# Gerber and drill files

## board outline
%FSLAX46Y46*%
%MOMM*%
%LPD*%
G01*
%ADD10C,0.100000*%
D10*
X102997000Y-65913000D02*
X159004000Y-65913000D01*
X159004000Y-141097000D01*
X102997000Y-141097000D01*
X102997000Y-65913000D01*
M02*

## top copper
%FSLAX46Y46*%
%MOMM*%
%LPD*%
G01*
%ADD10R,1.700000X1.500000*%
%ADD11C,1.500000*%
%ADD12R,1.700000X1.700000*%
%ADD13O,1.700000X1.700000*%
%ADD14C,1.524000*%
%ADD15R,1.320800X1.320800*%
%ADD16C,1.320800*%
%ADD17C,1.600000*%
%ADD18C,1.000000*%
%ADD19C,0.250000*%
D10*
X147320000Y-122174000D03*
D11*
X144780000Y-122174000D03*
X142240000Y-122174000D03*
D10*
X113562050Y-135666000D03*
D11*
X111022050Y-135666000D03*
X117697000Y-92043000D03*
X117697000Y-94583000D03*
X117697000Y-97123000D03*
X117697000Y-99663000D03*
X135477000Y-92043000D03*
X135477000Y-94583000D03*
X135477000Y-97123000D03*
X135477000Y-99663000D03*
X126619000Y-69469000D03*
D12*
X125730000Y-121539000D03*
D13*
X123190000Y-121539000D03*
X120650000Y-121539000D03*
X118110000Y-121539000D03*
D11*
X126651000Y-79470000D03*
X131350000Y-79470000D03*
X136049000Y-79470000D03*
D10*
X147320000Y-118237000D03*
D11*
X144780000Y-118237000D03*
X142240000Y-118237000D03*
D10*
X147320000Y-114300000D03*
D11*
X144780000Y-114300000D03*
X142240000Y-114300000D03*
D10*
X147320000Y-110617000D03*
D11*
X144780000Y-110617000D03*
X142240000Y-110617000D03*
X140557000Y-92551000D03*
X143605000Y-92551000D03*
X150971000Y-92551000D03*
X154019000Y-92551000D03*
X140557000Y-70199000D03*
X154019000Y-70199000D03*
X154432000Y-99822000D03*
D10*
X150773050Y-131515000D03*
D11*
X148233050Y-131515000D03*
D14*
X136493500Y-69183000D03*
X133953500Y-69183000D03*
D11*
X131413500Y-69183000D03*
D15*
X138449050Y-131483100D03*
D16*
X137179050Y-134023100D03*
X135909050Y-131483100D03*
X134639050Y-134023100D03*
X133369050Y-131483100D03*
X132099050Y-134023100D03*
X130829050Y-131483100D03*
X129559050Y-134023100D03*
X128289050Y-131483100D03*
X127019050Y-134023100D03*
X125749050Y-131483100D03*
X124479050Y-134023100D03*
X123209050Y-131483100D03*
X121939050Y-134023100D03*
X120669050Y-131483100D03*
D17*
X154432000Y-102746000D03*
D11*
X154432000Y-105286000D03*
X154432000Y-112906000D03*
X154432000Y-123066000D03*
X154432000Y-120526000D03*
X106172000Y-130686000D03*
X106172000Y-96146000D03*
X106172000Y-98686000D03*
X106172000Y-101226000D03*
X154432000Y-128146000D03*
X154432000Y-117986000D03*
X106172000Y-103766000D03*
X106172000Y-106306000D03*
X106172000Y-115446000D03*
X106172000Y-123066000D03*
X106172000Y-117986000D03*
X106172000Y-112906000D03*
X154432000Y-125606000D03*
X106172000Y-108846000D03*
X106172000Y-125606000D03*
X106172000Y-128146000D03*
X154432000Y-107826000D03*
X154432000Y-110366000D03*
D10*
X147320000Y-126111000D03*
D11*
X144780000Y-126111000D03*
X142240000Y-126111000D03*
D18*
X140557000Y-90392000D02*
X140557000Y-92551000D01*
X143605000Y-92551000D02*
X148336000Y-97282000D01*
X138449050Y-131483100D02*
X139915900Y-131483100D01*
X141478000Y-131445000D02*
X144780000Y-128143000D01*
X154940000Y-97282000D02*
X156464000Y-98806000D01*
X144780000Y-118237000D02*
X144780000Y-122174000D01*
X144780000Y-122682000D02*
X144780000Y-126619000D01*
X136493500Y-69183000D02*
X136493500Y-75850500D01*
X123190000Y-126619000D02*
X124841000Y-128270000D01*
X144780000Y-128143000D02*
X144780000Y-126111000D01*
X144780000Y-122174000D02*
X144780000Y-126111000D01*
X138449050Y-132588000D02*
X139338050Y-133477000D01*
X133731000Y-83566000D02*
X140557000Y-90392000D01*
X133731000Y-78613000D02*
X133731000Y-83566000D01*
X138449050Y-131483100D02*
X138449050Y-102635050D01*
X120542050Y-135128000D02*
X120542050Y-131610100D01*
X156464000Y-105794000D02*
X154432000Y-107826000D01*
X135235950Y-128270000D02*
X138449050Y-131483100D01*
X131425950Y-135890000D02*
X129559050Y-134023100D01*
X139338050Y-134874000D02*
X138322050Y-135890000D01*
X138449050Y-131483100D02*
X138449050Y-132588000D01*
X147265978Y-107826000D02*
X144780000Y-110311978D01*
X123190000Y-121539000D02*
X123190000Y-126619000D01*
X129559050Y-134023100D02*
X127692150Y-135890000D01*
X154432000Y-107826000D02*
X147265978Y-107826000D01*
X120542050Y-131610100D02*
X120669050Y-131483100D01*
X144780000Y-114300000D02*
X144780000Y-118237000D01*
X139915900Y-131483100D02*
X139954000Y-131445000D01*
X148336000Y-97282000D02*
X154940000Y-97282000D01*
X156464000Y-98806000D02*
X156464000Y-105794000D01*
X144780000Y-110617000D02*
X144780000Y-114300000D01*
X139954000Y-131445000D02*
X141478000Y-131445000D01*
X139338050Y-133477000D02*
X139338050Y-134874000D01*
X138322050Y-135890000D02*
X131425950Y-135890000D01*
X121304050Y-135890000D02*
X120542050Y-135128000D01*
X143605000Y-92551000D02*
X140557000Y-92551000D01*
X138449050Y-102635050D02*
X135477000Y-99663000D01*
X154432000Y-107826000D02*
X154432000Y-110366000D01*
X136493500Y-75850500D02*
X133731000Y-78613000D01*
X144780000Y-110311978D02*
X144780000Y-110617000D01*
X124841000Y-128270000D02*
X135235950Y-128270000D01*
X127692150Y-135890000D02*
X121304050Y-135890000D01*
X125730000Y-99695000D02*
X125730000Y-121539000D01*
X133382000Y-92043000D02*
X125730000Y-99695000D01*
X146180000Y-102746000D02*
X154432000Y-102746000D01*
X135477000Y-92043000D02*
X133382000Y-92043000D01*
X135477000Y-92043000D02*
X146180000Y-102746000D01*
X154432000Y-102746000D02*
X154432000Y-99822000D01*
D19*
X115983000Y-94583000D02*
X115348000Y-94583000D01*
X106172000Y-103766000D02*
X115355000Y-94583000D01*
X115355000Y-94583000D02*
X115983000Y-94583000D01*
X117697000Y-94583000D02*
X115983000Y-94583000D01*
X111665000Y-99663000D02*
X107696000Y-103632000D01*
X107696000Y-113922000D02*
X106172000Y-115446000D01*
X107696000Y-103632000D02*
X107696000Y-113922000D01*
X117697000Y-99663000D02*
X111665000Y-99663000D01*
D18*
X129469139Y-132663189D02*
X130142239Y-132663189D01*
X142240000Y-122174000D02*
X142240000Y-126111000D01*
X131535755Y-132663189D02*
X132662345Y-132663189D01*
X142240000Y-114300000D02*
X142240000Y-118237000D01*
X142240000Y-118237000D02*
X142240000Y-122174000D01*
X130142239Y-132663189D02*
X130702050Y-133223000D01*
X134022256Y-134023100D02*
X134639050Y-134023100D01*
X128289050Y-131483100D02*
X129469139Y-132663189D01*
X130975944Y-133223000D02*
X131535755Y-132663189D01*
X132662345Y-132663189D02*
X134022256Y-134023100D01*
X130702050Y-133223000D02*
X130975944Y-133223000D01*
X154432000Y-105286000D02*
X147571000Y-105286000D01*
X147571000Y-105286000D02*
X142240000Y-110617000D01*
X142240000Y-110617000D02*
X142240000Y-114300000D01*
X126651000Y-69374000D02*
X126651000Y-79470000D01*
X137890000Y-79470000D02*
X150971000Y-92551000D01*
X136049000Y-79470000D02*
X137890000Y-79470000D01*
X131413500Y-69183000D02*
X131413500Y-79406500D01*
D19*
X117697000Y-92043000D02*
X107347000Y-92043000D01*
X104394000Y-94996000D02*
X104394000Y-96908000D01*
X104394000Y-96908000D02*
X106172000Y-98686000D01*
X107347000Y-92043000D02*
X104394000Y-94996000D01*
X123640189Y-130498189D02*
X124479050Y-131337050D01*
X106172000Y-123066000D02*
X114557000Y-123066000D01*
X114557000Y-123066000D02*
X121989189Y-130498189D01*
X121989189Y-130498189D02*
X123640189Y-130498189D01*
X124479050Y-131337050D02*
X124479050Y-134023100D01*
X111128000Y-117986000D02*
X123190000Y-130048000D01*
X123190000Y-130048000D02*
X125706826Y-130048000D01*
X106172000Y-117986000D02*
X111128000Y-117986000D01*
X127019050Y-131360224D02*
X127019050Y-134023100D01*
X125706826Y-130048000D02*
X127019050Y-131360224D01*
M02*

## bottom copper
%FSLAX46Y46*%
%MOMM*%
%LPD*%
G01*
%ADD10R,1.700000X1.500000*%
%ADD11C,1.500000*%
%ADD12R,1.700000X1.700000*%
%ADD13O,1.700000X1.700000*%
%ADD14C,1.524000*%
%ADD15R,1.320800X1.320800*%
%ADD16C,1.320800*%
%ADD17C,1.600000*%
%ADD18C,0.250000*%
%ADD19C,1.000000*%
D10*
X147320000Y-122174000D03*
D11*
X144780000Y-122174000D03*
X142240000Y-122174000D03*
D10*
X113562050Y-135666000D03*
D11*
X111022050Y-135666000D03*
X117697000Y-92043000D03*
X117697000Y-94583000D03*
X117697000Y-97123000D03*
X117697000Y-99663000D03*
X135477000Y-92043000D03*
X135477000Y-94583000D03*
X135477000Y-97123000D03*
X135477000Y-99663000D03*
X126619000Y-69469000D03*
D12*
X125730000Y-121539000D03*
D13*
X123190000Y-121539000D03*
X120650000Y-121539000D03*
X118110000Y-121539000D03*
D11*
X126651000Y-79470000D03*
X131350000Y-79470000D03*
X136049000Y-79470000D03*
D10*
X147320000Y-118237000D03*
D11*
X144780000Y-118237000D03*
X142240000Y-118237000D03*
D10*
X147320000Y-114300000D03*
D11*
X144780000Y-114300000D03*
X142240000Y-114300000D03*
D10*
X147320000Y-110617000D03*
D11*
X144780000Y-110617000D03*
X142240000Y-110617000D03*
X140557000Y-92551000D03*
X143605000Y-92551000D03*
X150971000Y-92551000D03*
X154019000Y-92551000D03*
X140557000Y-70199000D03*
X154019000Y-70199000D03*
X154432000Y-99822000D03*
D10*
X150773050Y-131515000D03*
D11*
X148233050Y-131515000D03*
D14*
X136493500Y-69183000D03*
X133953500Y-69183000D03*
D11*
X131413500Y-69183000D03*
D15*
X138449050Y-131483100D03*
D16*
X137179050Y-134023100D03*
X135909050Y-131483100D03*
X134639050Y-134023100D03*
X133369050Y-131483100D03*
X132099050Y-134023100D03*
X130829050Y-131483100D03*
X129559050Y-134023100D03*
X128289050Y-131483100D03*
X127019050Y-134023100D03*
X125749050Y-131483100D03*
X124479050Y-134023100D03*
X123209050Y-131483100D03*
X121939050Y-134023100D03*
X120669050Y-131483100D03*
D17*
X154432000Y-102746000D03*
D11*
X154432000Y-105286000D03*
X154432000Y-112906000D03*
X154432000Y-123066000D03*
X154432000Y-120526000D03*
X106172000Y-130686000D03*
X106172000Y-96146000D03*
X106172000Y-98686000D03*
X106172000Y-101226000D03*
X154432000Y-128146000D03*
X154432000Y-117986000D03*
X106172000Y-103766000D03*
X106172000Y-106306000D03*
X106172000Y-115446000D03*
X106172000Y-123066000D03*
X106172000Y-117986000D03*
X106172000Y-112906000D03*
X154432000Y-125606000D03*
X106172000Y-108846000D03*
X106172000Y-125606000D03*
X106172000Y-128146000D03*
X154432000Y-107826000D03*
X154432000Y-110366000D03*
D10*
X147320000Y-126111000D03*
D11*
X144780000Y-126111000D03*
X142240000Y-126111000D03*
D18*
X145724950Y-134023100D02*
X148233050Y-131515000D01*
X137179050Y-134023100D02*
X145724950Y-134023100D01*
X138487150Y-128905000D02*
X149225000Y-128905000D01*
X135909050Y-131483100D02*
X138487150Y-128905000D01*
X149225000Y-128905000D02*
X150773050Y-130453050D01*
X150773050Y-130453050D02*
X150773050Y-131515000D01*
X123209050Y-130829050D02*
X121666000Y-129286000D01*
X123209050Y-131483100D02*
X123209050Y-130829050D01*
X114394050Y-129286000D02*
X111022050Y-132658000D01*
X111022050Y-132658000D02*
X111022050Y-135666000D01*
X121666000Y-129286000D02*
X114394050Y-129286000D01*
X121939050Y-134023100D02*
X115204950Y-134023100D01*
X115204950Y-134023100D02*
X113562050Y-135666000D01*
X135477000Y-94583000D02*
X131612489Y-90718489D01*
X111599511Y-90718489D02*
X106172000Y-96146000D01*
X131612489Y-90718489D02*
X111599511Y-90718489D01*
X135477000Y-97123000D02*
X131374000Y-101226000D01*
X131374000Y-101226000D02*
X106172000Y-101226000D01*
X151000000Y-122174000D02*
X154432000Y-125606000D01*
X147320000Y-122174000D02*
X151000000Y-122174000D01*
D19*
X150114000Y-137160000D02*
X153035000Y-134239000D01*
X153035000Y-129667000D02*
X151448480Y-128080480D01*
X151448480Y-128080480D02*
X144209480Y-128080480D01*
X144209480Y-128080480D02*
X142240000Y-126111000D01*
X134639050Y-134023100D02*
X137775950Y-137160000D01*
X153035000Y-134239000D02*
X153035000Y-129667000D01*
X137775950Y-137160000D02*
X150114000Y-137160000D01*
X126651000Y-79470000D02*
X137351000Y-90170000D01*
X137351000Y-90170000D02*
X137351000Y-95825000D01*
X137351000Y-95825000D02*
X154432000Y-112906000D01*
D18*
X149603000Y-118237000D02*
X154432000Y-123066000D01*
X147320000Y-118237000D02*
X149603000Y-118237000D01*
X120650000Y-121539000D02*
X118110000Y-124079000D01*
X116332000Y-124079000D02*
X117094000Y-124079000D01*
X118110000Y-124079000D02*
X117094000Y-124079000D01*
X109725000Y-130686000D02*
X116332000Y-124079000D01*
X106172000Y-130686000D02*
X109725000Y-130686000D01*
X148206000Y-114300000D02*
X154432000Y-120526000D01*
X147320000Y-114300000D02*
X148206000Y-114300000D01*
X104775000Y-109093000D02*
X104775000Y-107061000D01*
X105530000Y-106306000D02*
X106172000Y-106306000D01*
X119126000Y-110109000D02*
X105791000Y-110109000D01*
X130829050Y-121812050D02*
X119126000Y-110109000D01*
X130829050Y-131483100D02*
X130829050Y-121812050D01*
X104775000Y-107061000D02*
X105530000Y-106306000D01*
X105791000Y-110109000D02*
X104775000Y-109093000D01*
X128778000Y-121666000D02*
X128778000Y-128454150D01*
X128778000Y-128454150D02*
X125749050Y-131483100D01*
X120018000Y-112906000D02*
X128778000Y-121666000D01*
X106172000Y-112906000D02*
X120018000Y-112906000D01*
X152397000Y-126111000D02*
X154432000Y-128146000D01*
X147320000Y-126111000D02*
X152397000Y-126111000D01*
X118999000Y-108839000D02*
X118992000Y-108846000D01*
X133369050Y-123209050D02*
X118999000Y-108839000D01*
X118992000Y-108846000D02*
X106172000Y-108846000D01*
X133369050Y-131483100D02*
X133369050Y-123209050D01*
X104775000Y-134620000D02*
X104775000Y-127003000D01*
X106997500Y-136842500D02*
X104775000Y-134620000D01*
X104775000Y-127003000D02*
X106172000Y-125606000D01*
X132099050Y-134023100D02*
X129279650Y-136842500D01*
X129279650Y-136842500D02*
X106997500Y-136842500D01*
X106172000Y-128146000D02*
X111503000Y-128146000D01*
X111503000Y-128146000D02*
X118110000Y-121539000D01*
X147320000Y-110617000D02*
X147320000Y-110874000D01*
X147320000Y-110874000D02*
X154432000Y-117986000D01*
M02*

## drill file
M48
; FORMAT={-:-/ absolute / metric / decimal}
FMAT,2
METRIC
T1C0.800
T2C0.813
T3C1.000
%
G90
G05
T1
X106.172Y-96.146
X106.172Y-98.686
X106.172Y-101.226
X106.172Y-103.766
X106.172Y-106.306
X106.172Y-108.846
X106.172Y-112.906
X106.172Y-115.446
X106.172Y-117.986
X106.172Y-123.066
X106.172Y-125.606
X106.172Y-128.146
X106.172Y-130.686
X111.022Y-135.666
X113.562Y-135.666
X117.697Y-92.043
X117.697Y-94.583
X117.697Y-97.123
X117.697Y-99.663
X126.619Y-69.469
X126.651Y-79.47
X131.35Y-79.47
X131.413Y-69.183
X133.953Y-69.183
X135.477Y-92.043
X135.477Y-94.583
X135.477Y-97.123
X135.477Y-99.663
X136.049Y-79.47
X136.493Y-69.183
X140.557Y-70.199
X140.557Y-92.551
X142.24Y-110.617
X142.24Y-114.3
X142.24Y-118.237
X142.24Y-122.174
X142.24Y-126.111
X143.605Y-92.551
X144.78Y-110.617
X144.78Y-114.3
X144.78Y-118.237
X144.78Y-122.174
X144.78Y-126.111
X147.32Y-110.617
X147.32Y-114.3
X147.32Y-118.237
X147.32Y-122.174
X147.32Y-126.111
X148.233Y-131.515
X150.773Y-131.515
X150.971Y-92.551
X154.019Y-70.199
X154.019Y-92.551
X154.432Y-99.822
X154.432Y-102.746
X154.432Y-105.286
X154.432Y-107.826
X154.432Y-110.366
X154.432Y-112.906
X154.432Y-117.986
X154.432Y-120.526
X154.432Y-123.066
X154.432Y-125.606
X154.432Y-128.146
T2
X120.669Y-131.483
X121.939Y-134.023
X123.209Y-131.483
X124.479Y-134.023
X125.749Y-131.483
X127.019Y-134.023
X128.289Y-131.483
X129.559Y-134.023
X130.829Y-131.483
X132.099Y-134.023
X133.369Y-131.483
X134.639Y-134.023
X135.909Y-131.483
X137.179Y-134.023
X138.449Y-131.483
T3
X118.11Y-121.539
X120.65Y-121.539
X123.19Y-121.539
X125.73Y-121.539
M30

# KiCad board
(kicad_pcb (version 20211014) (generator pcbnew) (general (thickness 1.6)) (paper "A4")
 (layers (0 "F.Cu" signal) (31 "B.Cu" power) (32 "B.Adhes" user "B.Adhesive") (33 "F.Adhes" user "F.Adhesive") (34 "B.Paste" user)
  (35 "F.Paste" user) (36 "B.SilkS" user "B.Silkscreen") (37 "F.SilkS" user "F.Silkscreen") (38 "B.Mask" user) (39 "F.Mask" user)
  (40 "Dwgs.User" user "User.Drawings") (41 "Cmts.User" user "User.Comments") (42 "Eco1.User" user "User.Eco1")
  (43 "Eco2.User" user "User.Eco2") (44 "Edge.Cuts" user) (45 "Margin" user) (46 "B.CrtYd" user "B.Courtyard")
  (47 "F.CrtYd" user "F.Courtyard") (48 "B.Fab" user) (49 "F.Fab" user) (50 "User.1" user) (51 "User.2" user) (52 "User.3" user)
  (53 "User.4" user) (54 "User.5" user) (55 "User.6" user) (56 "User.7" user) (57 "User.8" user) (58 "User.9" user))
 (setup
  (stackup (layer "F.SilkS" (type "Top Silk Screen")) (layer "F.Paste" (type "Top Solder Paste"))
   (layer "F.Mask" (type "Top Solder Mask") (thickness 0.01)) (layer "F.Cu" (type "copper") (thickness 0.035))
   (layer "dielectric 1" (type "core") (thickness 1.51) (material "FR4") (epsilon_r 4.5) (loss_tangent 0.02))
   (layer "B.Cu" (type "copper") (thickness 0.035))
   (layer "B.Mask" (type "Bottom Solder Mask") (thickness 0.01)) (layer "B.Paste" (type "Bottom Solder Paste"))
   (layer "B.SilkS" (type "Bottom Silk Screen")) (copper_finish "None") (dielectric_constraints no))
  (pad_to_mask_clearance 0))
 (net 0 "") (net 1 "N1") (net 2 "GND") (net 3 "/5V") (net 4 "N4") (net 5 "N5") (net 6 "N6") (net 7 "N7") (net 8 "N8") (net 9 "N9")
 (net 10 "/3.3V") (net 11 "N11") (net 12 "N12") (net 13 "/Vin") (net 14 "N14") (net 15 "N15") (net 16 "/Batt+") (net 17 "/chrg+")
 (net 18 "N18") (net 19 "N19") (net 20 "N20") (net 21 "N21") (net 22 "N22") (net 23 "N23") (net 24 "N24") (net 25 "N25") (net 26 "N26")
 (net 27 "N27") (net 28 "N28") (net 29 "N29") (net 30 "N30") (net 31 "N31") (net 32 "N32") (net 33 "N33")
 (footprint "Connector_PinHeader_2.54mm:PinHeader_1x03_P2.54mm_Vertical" (layer "F.Cu") (at 147.32 122.174 -90)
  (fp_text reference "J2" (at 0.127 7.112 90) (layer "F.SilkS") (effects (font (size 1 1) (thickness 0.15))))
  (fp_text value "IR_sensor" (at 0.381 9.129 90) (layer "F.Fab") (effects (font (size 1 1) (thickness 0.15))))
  (pad "1" thru_hole rect (at 0 0 270) (size 1.5 1.7) (drill 0.8) (layers *.Cu *.Mask) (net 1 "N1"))
  (pad "2" thru_hole circle (at 0 2.54 270) (size 1.5 1.5) (drill 0.8) (layers *.Cu *.Mask) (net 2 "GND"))
  (pad "3" thru_hole circle (at 0 5.08 270) (size 1.5 1.5) (drill 0.8) (layers *.Cu *.Mask) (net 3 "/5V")))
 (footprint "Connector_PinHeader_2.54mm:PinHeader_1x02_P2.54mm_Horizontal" (layer "F.Cu") (at 113.56205 135.666 -90)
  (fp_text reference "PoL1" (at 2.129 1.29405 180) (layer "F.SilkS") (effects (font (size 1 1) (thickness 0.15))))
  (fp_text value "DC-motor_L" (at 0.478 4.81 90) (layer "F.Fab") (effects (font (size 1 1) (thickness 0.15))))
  (pad "1" thru_hole rect (at 0 0 270) (size 1.5 1.7) (drill 0.8) (layers *.Cu *.Mask) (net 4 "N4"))
  (pad "2" thru_hole circle (at 0 2.54 270) (size 1.5 1.5) (drill 0.8) (layers *.Cu *.Mask) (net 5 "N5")))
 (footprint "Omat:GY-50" (layer "F.Cu") (at 115.03 84.296 -90)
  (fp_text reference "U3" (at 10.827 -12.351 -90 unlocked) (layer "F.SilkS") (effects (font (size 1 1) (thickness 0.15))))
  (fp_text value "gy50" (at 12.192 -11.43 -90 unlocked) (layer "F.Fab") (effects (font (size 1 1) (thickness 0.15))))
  (pad "1" thru_hole circle (at 7.747 -2.667 270) (size 1.5 1.5) (drill 0.8) (layers *.Cu *.Mask) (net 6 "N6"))
  (pad "2" thru_hole circle (at 10.287 -2.667 270) (size 1.5 1.5) (drill 0.8) (layers *.Cu *.Mask) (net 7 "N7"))
  (pad "3" thru_hole circle (at 12.827 -2.667 270) (size 1.5 1.5) (drill 0.8) (layers *.Cu *.Mask) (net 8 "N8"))
  (pad "4" thru_hole circle (at 15.367 -2.667 270) (size 1.5 1.5) (drill 0.8) (layers *.Cu *.Mask) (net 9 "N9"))
  (pad "5" thru_hole circle (at 7.747 -20.447 270) (size 1.5 1.5) (drill 0.8) (layers *.Cu *.Mask) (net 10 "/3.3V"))
  (pad "6" thru_hole circle (at 10.287 -20.447 270) (size 1.5 1.5) (drill 0.8) (layers *.Cu *.Mask) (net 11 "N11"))
  (pad "7" thru_hole circle (at 12.827 -20.447 270) (size 1.5 1.5) (drill 0.8) (layers *.Cu *.Mask) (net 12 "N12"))
  (pad "8" thru_hole circle (at 15.367 -20.447 270) (size 1.5 1.5) (drill 0.8) (layers *.Cu *.Mask) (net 2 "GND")))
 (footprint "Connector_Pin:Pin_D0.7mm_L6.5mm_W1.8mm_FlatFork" (layer "F.Cu") (at 126.619 69.469)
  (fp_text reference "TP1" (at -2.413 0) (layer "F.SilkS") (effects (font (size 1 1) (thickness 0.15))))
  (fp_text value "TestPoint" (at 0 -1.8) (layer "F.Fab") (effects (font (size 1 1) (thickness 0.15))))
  (pad "1" thru_hole circle (at 0 0) (size 1.5 1.5) (drill 0.8) (layers *.Cu *.Mask) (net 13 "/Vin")))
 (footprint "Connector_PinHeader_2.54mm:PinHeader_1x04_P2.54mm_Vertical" (layer "F.Cu") (at 125.73 121.539 -90)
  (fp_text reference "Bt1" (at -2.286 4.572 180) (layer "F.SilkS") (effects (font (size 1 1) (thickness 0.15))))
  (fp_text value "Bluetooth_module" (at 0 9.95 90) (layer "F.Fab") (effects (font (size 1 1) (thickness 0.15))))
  (pad "1" thru_hole rect (at 0 0 270) (size 1.7 1.7) (drill 1) (layers *.Cu *.Mask) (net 10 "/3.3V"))
  (pad "2" thru_hole oval (at 0 2.54 270) (size 1.7 1.7) (drill 1) (layers *.Cu *.Mask) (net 2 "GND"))
  (pad "3" thru_hole oval (at 0 5.08 270) (size 1.7 1.7) (drill 1) (layers *.Cu *.Mask) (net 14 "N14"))
  (pad "4" thru_hole oval (at 0 7.62 270) (size 1.7 1.7) (drill 1) (layers *.Cu *.Mask) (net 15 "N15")))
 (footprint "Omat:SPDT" (layer "F.Cu") (at 137.954 75.406 180)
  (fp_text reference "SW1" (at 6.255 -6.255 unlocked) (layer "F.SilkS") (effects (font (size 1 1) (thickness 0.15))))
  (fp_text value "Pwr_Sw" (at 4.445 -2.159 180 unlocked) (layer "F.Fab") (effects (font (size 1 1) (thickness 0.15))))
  (pad "1" thru_hole circle (at 11.303 -4.064 180) (size 1.5 1.5) (drill 0.8) (layers *.Cu *.Mask) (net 13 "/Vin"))
  (pad "2" thru_hole circle (at 6.604 -4.064 180) (size 1.5 1.5) (drill 0.8) (layers *.Cu *.Mask) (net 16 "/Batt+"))
  (pad "3" thru_hole circle (at 1.905 -4.064 180) (size 1.5 1.5) (drill 0.8) (layers *.Cu *.Mask) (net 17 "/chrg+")))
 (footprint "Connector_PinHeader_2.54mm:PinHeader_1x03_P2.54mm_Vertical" (layer "F.Cu") (at 147.32 118.237 -90)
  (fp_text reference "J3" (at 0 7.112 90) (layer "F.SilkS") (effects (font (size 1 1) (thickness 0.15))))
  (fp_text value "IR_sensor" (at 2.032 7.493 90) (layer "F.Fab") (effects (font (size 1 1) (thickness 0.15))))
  (pad "1" thru_hole rect (at 0 0 270) (size 1.5 1.7) (drill 0.8) (layers *.Cu *.Mask) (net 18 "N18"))
  (pad "2" thru_hole circle (at 0 2.54 270) (size 1.5 1.5) (drill 0.8) (layers *.Cu *.Mask) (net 2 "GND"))
  (pad "3" thru_hole circle (at 0 5.08 270) (size 1.5 1.5) (drill 0.8) (layers *.Cu *.Mask) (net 3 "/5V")))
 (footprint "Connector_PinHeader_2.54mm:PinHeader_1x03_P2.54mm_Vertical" (layer "F.Cu") (at 147.32 114.3 -90)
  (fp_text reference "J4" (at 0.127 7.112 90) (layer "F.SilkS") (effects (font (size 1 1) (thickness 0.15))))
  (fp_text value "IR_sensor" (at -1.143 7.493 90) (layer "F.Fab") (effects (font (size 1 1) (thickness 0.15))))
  (pad "1" thru_hole rect (at 0 0 270) (size 1.5 1.7) (drill 0.8) (layers *.Cu *.Mask) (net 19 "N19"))
  (pad "2" thru_hole circle (at 0 2.54 270) (size 1.5 1.5) (drill 0.8) (layers *.Cu *.Mask) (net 2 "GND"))
  (pad "3" thru_hole circle (at 0 5.08 270) (size 1.5 1.5) (drill 0.8) (layers *.Cu *.Mask) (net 3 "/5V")))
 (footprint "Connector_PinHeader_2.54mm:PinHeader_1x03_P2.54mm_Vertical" (layer "F.Cu") (at 147.32 110.617 -90)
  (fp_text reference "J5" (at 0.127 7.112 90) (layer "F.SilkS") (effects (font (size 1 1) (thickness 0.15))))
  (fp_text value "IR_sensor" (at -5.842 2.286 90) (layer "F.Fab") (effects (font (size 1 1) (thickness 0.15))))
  (pad "1" thru_hole rect (at 0 0 270) (size 1.5 1.7) (drill 0.8) (layers *.Cu *.Mask) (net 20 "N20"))
  (pad "2" thru_hole circle (at 0 2.54 270) (size 1.5 1.5) (drill 0.8) (layers *.Cu *.Mask) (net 2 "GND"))
  (pad "3" thru_hole circle (at 0 5.08 270) (size 1.5 1.5) (drill 0.8) (layers *.Cu *.Mask) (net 3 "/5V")))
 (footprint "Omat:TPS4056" (layer "F.Cu") (at 138.779 67.659 -90)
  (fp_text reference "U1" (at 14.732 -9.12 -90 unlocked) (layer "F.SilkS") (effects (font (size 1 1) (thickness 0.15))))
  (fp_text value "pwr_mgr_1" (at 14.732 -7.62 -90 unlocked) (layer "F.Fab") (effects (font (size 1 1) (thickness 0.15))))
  (pad "1" thru_hole circle (at 24.892 -1.778 270) (size 1.5 1.5) (drill 0.8) (layers *.Cu *.Mask) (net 2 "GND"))
  (pad "2" thru_hole circle (at 24.892 -4.826 270) (size 1.5 1.5) (drill 0.8) (layers *.Cu *.Mask) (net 2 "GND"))
  (pad "3" thru_hole circle (at 24.892 -12.192 270) (size 1.5 1.5) (drill 0.8) (layers *.Cu *.Mask) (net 17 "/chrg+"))
  (pad "4" thru_hole circle (at 24.892 -15.24 270) (size 1.5 1.5) (drill 0.8) (layers *.Cu *.Mask) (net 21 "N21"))
  (pad "5" thru_hole circle (at 2.54 -1.778 270) (size 1.5 1.5) (drill 0.8) (layers *.Cu *.Mask) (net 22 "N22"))
  (pad "6" thru_hole circle (at 2.54 -15.24 270) (size 1.5 1.5) (drill 0.8) (layers *.Cu *.Mask) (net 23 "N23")))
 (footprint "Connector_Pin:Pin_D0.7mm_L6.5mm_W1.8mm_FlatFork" (layer "F.Cu") (at 154.432 99.822)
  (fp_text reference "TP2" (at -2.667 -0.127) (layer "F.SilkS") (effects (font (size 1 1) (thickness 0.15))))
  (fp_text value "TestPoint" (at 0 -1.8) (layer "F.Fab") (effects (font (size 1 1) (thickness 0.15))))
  (pad "1" thru_hole circle (at 0 0) (size 1.5 1.5) (drill 0.8) (layers *.Cu *.Mask) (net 10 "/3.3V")))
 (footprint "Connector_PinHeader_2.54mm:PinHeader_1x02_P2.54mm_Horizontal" (layer "F.Cu") (at 150.77305 131.515 -90)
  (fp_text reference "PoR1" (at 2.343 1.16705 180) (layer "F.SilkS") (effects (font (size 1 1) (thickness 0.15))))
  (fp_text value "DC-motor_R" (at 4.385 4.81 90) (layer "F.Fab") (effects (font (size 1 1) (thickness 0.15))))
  (pad "1" thru_hole rect (at 0 0 270) (size 1.5 1.7) (drill 0.8) (layers *.Cu *.Mask) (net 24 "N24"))
  (pad "2" thru_hole circle (at 0 2.54 270) (size 1.5 1.5) (drill 0.8) (layers *.Cu *.Mask) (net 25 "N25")))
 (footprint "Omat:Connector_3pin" (layer "F.Cu") (at 137.6365 67.913 180)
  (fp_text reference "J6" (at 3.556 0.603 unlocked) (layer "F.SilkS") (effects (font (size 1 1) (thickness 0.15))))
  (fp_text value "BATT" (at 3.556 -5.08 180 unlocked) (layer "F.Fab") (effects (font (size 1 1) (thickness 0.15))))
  (pad "1" thru_hole circle (at 1.143 -1.27 180) (size 1.524 1.524) (drill 0.8) (layers *.Cu *.Mask) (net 2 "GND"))
  (pad "2" thru_hole circle (at 3.683 -1.27 180) (size 1.524 1.524) (drill 0.8) (layers *.Cu *.Mask) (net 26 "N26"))
  (pad "3" thru_hole circle (at 6.223 -1.27 180) (size 1.5 1.5) (drill 0.8) (layers *.Cu *.Mask) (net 16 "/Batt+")))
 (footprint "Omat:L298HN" (layer "F.Cu") (at 138.44905 131.4831 180)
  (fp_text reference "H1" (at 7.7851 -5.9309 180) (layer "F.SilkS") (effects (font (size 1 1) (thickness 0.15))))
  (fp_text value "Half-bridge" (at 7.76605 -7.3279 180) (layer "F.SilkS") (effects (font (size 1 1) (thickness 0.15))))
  (pad "1" thru_hole rect (at 0 0 180) (size 1.3208 1.3208) (drill 0.8128) (layers *.Cu *.Mask) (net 2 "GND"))
  (pad "2" thru_hole circle (at 1.27 -2.54 180) (size 1.3208 1.3208) (drill 0.8128) (layers *.Cu *.Mask) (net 25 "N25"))
  (pad "3" thru_hole circle (at 2.54 0 180) (size 1.3208 1.3208) (drill 0.8128) (layers *.Cu *.Mask) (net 24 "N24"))
  (pad "4" thru_hole circle (at 3.81 -2.54 180) (size 1.3208 1.3208) (drill 0.8128) (layers *.Cu *.Mask) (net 3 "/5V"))
  (pad "5" thru_hole circle (at 5.08 0 180) (size 1.3208 1.3208) (drill 0.8128) (layers *.Cu *.Mask) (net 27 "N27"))
  (pad "6" thru_hole circle (at 6.35 -2.54 180) (size 1.3208 1.3208) (drill 0.8128) (layers *.Cu *.Mask) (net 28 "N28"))
  (pad "7" thru_hole circle (at 7.62 0 180) (size 1.3208 1.3208) (drill 0.8128) (layers *.Cu *.Mask) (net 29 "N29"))
  (pad "8" thru_hole circle (at 8.89 -2.54 180) (size 1.3208 1.3208) (drill 0.8128) (layers *.Cu *.Mask) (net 2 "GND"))
  (pad "9" thru_hole circle (at 10.16 0 180) (size 1.3208 1.3208) (drill 0.8128) (layers *.Cu *.Mask) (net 3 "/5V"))
  (pad "10" thru_hole circle (at 11.43 -2.54 180) (size 1.3208 1.3208) (drill 0.8128) (layers *.Cu *.Mask) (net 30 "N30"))
  (pad "11" thru_hole circle (at 12.7 0 180) (size 1.3208 1.3208) (drill 0.8128) (layers *.Cu *.Mask) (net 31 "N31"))
  (pad "12" thru_hole circle (at 13.97 -2.54 180) (size 1.3208 1.3208) (drill 0.8128) (layers *.Cu *.Mask) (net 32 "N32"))
  (pad "13" thru_hole circle (at 15.24 0 180) (size 1.3208 1.3208) (drill 0.8128) (layers *.Cu *.Mask) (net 5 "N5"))
  (pad "14" thru_hole circle (at 16.51 -2.54 180) (size 1.3208 1.3208) (drill 0.8128) (layers *.Cu *.Mask) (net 4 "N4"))
  (pad "15" thru_hole circle (at 17.78 0 180) (size 1.3208 1.3208) (drill 0.8128) (layers *.Cu *.Mask) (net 2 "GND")))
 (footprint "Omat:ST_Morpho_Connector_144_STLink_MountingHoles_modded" (layer "F.Cu") (at 98.679 67.313)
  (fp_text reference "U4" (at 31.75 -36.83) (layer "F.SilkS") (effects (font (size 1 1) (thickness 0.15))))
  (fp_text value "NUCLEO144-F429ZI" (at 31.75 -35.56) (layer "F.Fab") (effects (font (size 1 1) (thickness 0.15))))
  (pad "16" thru_hole circle (at 55.753 35.433) (size 1.6 1.6) (drill 0.8) (layers *.Cu *.Mask) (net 10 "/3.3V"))
  (pad "18" thru_hole circle (at 55.753 37.973) (size 1.5 1.5) (drill 0.8) (layers *.Cu *.Mask) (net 3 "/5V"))
  (pad "24" thru_hole circle (at 55.753 45.593) (size 1.5 1.5) (drill 0.8) (layers *.Cu *.Mask) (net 13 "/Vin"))
  (pad "37" thru_hole circle (at 55.753 55.753) (size 1.5 1.5) (drill 0.8) (layers *.Cu *.Mask) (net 18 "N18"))
  (pad "38" thru_hole circle (at 55.753 53.213) (size 1.5 1.5) (drill 0.8) (layers *.Cu *.Mask) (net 19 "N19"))
  (pad "63" thru_hole circle (at 7.493 63.373) (size 1.5 1.5) (drill 0.8) (layers *.Cu *.Mask) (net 14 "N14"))
  (pad "83" thru_hole circle (at 7.493 28.833) (size 1.5 1.5) (drill 0.8) (layers *.Cu *.Mask) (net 11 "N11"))
  (pad "85" thru_hole circle (at 7.493 31.373) (size 1.5 1.5) (drill 0.8) (layers *.Cu *.Mask) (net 6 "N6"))
  (pad "87" thru_hole circle (at 7.493 33.913) (size 1.5 1.5) (drill 0.8) (layers *.Cu *.Mask) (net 12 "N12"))
  (pad "108" thru_hole circle (at 55.753 60.833) (size 1.5 1.5) (drill 0.8) (layers *.Cu *.Mask) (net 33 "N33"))
  (pad "114" thru_hole circle (at 55.753 50.673) (size 1.5 1.5) (drill 0.8) (layers *.Cu *.Mask) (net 20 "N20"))
  (pad "118" thru_hole circle (at 7.493 36.453) (size 1.5 1.5) (drill 0.8) (layers *.Cu *.Mask) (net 7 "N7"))
  (pad "120" thru_hole circle (at 7.493 38.993) (size 1.5 1.5) (drill 0.8) (layers *.Cu *.Mask) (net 29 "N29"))
  (pad "124" thru_hole circle (at 7.493 48.133) (size 1.5 1.5) (drill 0.8) (layers *.Cu *.Mask) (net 9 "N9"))
  (pad "127" thru_hole circle (at 7.493 55.753) (size 1.5 1.5) (drill 0.8) (layers *.Cu *.Mask) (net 32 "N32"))
  (pad "128" thru_hole circle (at 7.493 50.673) (size 1.5 1.5) (drill 0.8) (layers *.Cu *.Mask) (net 30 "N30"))
  (pad "129" thru_hole circle (at 7.493 45.593) (size 1.5 1.5) (drill 0.8) (layers *.Cu *.Mask) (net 31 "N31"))
  (pad "130" thru_hole circle (at 55.753 58.293) (size 1.5 1.5) (drill 0.8) (layers *.Cu *.Mask) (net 1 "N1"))
  (pad "131" thru_hole circle (at 7.493 41.533) (size 1.5 1.5) (drill 0.8) (layers *.Cu *.Mask) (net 27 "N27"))
  (pad "132" thru_hole circle (at 7.493 58.293) (size 1.5 1.5) (drill 0.8) (layers *.Cu *.Mask) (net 28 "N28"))
  (pad "133" thru_hole circle (at 7.493 60.833) (size 1.5 1.5) (drill 0.8) (layers *.Cu *.Mask) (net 15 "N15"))
  (pad "143" thru_hole circle (at 55.753 40.513) (size 1.5 1.5) (drill 0.8) (layers *.Cu *.Mask) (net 2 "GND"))
  (pad "144" thru_hole circle (at 55.753 43.053) (size 1.5 1.5) (drill 0.8) (layers *.Cu *.Mask) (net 2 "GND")))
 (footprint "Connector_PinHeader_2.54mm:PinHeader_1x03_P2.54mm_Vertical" (layer "F.Cu") (at 147.32 126.111 -90)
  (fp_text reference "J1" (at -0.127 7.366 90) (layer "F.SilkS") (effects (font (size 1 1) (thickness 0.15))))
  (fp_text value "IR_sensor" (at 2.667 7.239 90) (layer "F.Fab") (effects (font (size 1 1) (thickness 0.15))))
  (pad "1" thru_hole rect (at 0 0 270) (size 1.5 1.7) (drill 0.8) (layers *.Cu *.Mask) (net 33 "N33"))
  (pad "2" thru_hole circle (at 0 2.54 270) (size 1.5 1.5) (drill 0.8) (layers *.Cu *.Mask) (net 2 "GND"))
  (pad "3" thru_hole circle (at 0 5.08 270) (size 1.5 1.5) (drill 0.8) (layers *.Cu *.Mask) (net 3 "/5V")))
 (gr_rect (start 102.997 65.913) (end 159.004 141.097) (layer "Edge.Cuts") (width 0.1) (fill none))
 (segment (start 140.557 90.392) (end 140.557 92.551) (width 1) (layer "F.Cu") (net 2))
 (segment (start 143.605 92.551) (end 148.336 97.282) (width 1) (layer "F.Cu") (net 2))
 (segment (start 138.44905 131.4831) (end 139.9159 131.4831) (width 1) (layer "F.Cu") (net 2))
 (segment (start 141.478 131.445) (end 144.78 128.143) (width 1) (layer "F.Cu") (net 2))
 (segment (start 154.94 97.282) (end 156.464 98.806) (width 1) (layer "F.Cu") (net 2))
 (segment (start 144.78 118.237) (end 144.78 122.174) (width 1) (layer "F.Cu") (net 2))
 (segment (start 144.78 122.682) (end 144.78 126.619) (width 1) (layer "F.Cu") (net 2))
 (segment (start 136.4935 69.183) (end 136.4935 75.8505) (width 1) (layer "F.Cu") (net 2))
 (segment (start 123.19 126.619) (end 124.841 128.27) (width 1) (layer "F.Cu") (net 2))
 (segment (start 144.78 128.143) (end 144.78 126.111) (width 1) (layer "F.Cu") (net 2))
 (segment (start 144.78 122.174) (end 144.78 126.111) (width 1) (layer "F.Cu") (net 2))
 (segment (start 138.44905 132.588) (end 139.33805 133.477) (width 1) (layer "F.Cu") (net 2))
 (segment (start 133.731 83.566) (end 140.557 90.392) (width 1) (layer "F.Cu") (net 2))
 (segment (start 133.731 78.613) (end 133.731 83.566) (width 1) (layer "F.Cu") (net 2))
 (segment (start 138.44905 131.4831) (end 138.44905 102.63505) (width 1) (layer "F.Cu") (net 2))
 (segment (start 120.54205 135.128) (end 120.54205 131.6101) (width 1) (layer "F.Cu") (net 2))
 (segment (start 156.464 105.794) (end 154.432 107.826) (width 1) (layer "F.Cu") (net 2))
 (segment (start 135.23595 128.27) (end 138.44905 131.4831) (width 1) (layer "F.Cu") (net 2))
 (segment (start 131.42595 135.89) (end 129.55905 134.0231) (width 1) (layer "F.Cu") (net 2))
 (segment (start 139.33805 134.874) (end 138.32205 135.89) (width 1) (layer "F.Cu") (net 2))
 (segment (start 138.44905 131.4831) (end 138.44905 132.588) (width 1) (layer "F.Cu") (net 2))
 (segment (start 147.265978 107.826) (end 144.78 110.311978) (width 1) (layer "F.Cu") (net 2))
 (segment (start 123.19 121.539) (end 123.19 126.619) (width 1) (layer "F.Cu") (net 2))
 (segment (start 129.55905 134.0231) (end 127.69215 135.89) (width 1) (layer "F.Cu") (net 2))
 (segment (start 154.432 107.826) (end 147.265978 107.826) (width 1) (layer "F.Cu") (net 2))
 (segment (start 120.54205 131.6101) (end 120.66905 131.4831) (width 1) (layer "F.Cu") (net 2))
 (segment (start 144.78 114.3) (end 144.78 118.237) (width 1) (layer "F.Cu") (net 2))
 (segment (start 139.9159 131.4831) (end 139.954 131.445) (width 1) (layer "F.Cu") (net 2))
 (segment (start 148.336 97.282) (end 154.94 97.282) (width 1) (layer "F.Cu") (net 2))
 (segment (start 156.464 98.806) (end 156.464 105.794) (width 1) (layer "F.Cu") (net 2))
 (segment (start 144.78 110.617) (end 144.78 114.3) (width 1) (layer "F.Cu") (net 2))
 (segment (start 139.954 131.445) (end 141.478 131.445) (width 1) (layer "F.Cu") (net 2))
 (segment (start 139.33805 133.477) (end 139.33805 134.874) (width 1) (layer "F.Cu") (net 2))
 (segment (start 138.32205 135.89) (end 131.42595 135.89) (width 1) (layer "F.Cu") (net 2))
 (segment (start 121.30405 135.89) (end 120.54205 135.128) (width 1) (layer "F.Cu") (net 2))
 (segment (start 143.605 92.551) (end 140.557 92.551) (width 1) (layer "F.Cu") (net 2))
 (segment (start 138.44905 102.63505) (end 135.477 99.663) (width 1) (layer "F.Cu") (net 2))
 (segment (start 154.432 107.826) (end 154.432 110.366) (width 1) (layer "F.Cu") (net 2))
 (segment (start 136.4935 75.8505) (end 133.731 78.613) (width 1) (layer "F.Cu") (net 2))
 (segment (start 144.78 110.311978) (end 144.78 110.617) (width 1) (layer "F.Cu") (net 2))
 (segment (start 124.841 128.27) (end 135.23595 128.27) (width 1) (layer "F.Cu") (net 2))
 (segment (start 127.69215 135.89) (end 121.30405 135.89) (width 1) (layer "F.Cu") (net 2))
 (segment (start 145.72495 134.0231) (end 148.23305 131.515) (width 0.25) (layer "B.Cu") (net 25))
 (segment (start 137.17905 134.0231) (end 145.72495 134.0231) (width 0.25) (layer "B.Cu") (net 25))
 (segment (start 138.48715 128.905) (end 149.225 128.905) (width 0.25) (layer "B.Cu") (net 24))
 (segment (start 135.90905 131.4831) (end 138.48715 128.905) (width 0.25) (layer "B.Cu") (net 24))
 (segment (start 149.225 128.905) (end 150.77305 130.45305) (width 0.25) (layer "B.Cu") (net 24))
 (segment (start 150.77305 130.45305) (end 150.77305 131.515) (width 0.25) (layer "B.Cu") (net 24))
 (segment (start 125.73 99.695) (end 125.73 121.539) (width 1) (layer "F.Cu") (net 10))
 (segment (start 133.382 92.043) (end 125.73 99.695) (width 1) (layer "F.Cu") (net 10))
 (segment (start 146.18 102.746) (end 154.432 102.746) (width 1) (layer "F.Cu") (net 10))
 (segment (start 135.477 92.043) (end 133.382 92.043) (width 1) (layer "F.Cu") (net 10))
 (segment (start 135.477 92.043) (end 146.18 102.746) (width 1) (layer "F.Cu") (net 10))
 (segment (start 154.432 102.746) (end 154.432 99.822) (width 1) (layer "F.Cu") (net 10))
 (segment (start 123.20905 130.82905) (end 121.666 129.286) (width 0.25) (layer "B.Cu") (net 5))
 (segment (start 123.20905 131.4831) (end 123.20905 130.82905) (width 0.25) (layer "B.Cu") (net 5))
 (segment (start 114.39405 129.286) (end 111.02205 132.658) (width 0.25) (layer "B.Cu") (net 5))
 (segment (start 111.02205 132.658) (end 111.02205 135.666) (width 0.25) (layer "B.Cu") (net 5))
 (segment (start 121.666 129.286) (end 114.39405 129.286) (width 0.25) (layer "B.Cu") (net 5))
 (segment (start 121.93905 134.0231) (end 115.20495 134.0231) (width 0.25) (layer "B.Cu") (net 4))
 (segment (start 115.20495 134.0231) (end 113.56205 135.666) (width 0.25) (layer "B.Cu") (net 4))
 (segment (start 115.983 94.583) (end 115.348 94.583) (width 0.25) (layer "F.Cu") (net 7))
 (segment (start 106.172 103.766) (end 115.355 94.583) (width 0.25) (layer "F.Cu") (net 7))
 (segment (start 115.355 94.583) (end 115.983 94.583) (width 0.25) (layer "F.Cu") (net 7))
 (segment (start 117.697 94.583) (end 115.983 94.583) (width 0.25) (layer "F.Cu") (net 7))
 (segment (start 111.665 99.663) (end 107.696 103.632) (width 0.25) (layer "F.Cu") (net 9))
 (segment (start 107.696 113.922) (end 106.172 115.446) (width 0.25) (layer "F.Cu") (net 9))
 (segment (start 107.696 103.632) (end 107.696 113.922) (width 0.25) (layer "F.Cu") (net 9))
 (segment (start 117.697 99.663) (end 111.665 99.663) (width 0.25) (layer "F.Cu") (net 9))
 (segment (start 135.477 94.583) (end 131.612489 90.718489) (width 0.25) (layer "B.Cu") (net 11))
 (segment (start 111.599511 90.718489) (end 106.172 96.146) (width 0.25) (layer "B.Cu") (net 11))
 (segment (start 131.612489 90.718489) (end 111.599511 90.718489) (width 0.25) (layer "B.Cu") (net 11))
 (segment (start 135.477 97.123) (end 131.374 101.226) (width 0.25) (layer "B.Cu") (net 12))
 (segment (start 131.374 101.226) (end 106.172 101.226) (width 0.25) (layer "B.Cu") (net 12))
 (segment (start 151 122.174) (end 154.432 125.606) (width 0.25) (layer "B.Cu") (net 1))
 (segment (start 147.32 122.174) (end 151 122.174) (width 0.25) (layer "B.Cu") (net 1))
 (segment (start 129.469139 132.663189) (end 130.142239 132.663189) (width 1) (layer "F.Cu") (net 3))
 (segment (start 142.24 122.174) (end 142.24 126.111) (width 1) (layer "F.Cu") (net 3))
 (segment (start 131.535755 132.663189) (end 132.662345 132.663189) (width 1) (layer "F.Cu") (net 3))
 (segment (start 142.24 114.3) (end 142.24 118.237) (width 1) (layer "F.Cu") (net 3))
 (segment (start 142.24 118.237) (end 142.24 122.174) (width 1) (layer "F.Cu") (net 3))
 (segment (start 130.142239 132.663189) (end 130.70205 133.223) (width 1) (layer "F.Cu") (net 3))
 (segment (start 134.022256 134.0231) (end 134.63905 134.0231) (width 1) (layer "F.Cu") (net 3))
 (segment (start 128.28905 131.4831) (end 129.469139 132.663189) (width 1) (layer "F.Cu") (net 3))
 (segment (start 130.975944 133.223) (end 131.535755 132.663189) (width 1) (layer "F.Cu") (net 3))
 (segment (start 132.662345 132.663189) (end 134.022256 134.0231) (width 1) (layer "F.Cu") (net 3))
 (segment (start 130.70205 133.223) (end 130.975944 133.223) (width 1) (layer "F.Cu") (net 3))
 (segment (start 154.432 105.286) (end 147.571 105.286) (width 1) (layer "F.Cu") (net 3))
 (segment (start 147.571 105.286) (end 142.24 110.617) (width 1) (layer "F.Cu") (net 3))
 (segment (start 142.24 110.617) (end 142.24 114.3) (width 1) (layer "F.Cu") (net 3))
 (segment (start 150.114 137.16) (end 153.035 134.239) (width 1) (layer "B.Cu") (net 3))
 (segment (start 153.035 129.667) (end 151.44848 128.08048) (width 1) (layer "B.Cu") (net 3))
 (segment (start 151.44848 128.08048) (end 144.20948 128.08048) (width 1) (layer "B.Cu") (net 3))
 (segment (start 144.20948 128.08048) (end 142.24 126.111) (width 1) (layer "B.Cu") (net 3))
 (segment (start 134.63905 134.0231) (end 137.77595 137.16) (width 1) (layer "B.Cu") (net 3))
 (segment (start 153.035 134.239) (end 153.035 129.667) (width 1) (layer "B.Cu") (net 3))
 (segment (start 137.77595 137.16) (end 150.114 137.16) (width 1) (layer "B.Cu") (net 3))
 (segment (start 126.651 69.374) (end 126.651 79.47) (width 1) (layer "F.Cu") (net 13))
 (segment (start 126.651 79.47) (end 137.351 90.17) (width 1) (layer "B.Cu") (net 13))
 (segment (start 137.351 90.17) (end 137.351 95.825) (width 1) (layer "B.Cu") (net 13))
 (segment (start 137.351 95.825) (end 154.432 112.906) (width 1) (layer "B.Cu") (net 13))
 (segment (start 137.89 79.47) (end 150.971 92.551) (width 1) (layer "F.Cu") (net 17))
 (segment (start 136.049 79.47) (end 137.89 79.47) (width 1) (layer "F.Cu") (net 17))
 (segment (start 131.4135 69.183) (end 131.4135 79.4065) (width 1) (layer "F.Cu") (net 16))
 (segment (start 149.603 118.237) (end 154.432 123.066) (width 0.25) (layer "B.Cu") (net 18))
 (segment (start 147.32 118.237) (end 149.603 118.237) (width 0.25) (layer "B.Cu") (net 18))
 (segment (start 120.65 121.539) (end 118.11 124.079) (width 0.25) (layer "B.Cu") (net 14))
 (segment (start 116.332 124.079) (end 117.094 124.079) (width 0.25) (layer "B.Cu") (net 14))
 (segment (start 118.11 124.079) (end 117.094 124.079) (width 0.25) (layer "B.Cu") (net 14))
 (segment (start 109.725 130.686) (end 116.332 124.079) (width 0.25) (layer "B.Cu") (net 14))
 (segment (start 106.172 130.686) (end 109.725 130.686) (width 0.25) (layer "B.Cu") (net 14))
 (segment (start 117.697 92.043) (end 107.347 92.043) (width 0.25) (layer "F.Cu") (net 6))
 (segment (start 104.394 94.996) (end 104.394 96.908) (width 0.25) (layer "F.Cu") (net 6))
 (segment (start 104.394 96.908) (end 106.172 98.686) (width 0.25) (layer "F.Cu") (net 6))
 (segment (start 107.347 92.043) (end 104.394 94.996) (width 0.25) (layer "F.Cu") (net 6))
 (segment (start 148.206 114.3) (end 154.432 120.526) (width 0.25) (layer "B.Cu") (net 19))
 (segment (start 147.32 114.3) (end 148.206 114.3) (width 0.25) (layer "B.Cu") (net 19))
 (segment (start 104.775 109.093) (end 104.775 107.061) (width 0.25) (layer "B.Cu") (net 29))
 (segment (start 105.53 106.306) (end 106.172 106.306) (width 0.25) (layer "B.Cu") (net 29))
 (segment (start 119.126 110.109) (end 105.791 110.109) (width 0.25) (layer "B.Cu") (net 29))
 (segment (start 130.82905 121.81205) (end 119.126 110.109) (width 0.25) (layer "B.Cu") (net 29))
 (segment (start 130.82905 131.4831) (end 130.82905 121.81205) (width 0.25) (layer "B.Cu") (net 29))
 (segment (start 104.775 107.061) (end 105.53 106.306) (width 0.25) (layer "B.Cu") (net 29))
 (segment (start 105.791 110.109) (end 104.775 109.093) (width 0.25) (layer "B.Cu") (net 29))
 (segment (start 123.640189 130.498189) (end 124.47905 131.33705) (width 0.25) (layer "F.Cu") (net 32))
 (segment (start 106.172 123.066) (end 114.557 123.066) (width 0.25) (layer "F.Cu") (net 32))
 (segment (start 114.557 123.066) (end 121.989189 130.498189) (width 0.25) (layer "F.Cu") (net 32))
 (segment (start 121.989189 130.498189) (end 123.640189 130.498189) (width 0.25) (layer "F.Cu") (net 32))
 (segment (start 124.47905 131.33705) (end 124.47905 134.0231) (width 0.25) (layer "F.Cu") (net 32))
 (segment (start 111.128 117.986) (end 123.19 130.048) (width 0.25) (layer "F.Cu") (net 30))
 (segment (start 123.19 130.048) (end 125.706826 130.048) (width 0.25) (layer "F.Cu") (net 30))
 (segment (start 106.172 117.986) (end 111.128 117.986) (width 0.25) (layer "F.Cu") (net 30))
 (segment (start 127.01905 131.360224) (end 127.01905 134.0231) (width 0.25) (layer "F.Cu") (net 30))
 (segment (start 125.706826 130.048) (end 127.01905 131.360224) (width 0.25) (layer "F.Cu") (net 30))
 (segment (start 128.778 121.666) (end 128.778 128.45415) (width 0.25) (layer "B.Cu") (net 31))
 (segment (start 128.778 128.45415) (end 125.74905 131.4831) (width 0.25) (layer "B.Cu") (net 31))
 (segment (start 120.018 112.906) (end 128.778 121.666) (width 0.25) (layer "B.Cu") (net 31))
 (segment (start 106.172 112.906) (end 120.018 112.906) (width 0.25) (layer "B.Cu") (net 31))
 (segment (start 152.397 126.111) (end 154.432 128.146) (width 0.25) (layer "B.Cu") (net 33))
 (segment (start 147.32 126.111) (end 152.397 126.111) (width 0.25) (layer "B.Cu") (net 33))
 (segment (start 118.999 108.839) (end 118.992 108.846) (width 0.25) (layer "B.Cu") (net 27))
 (segment (start 133.36905 123.20905) (end 118.999 108.839) (width 0.25) (layer "B.Cu") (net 27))
 (segment (start 118.992 108.846) (end 106.172 108.846) (width 0.25) (layer "B.Cu") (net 27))
 (segment (start 133.36905 131.4831) (end 133.36905 123.20905) (width 0.25) (layer "B.Cu") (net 27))
 (segment (start 104.775 134.62) (end 104.775 127.003) (width 0.25) (layer "B.Cu") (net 28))
 (segment (start 106.9975 136.8425) (end 104.775 134.62) (width 0.25) (layer "B.Cu") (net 28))
 (segment (start 104.775 127.003) (end 106.172 125.606) (width 0.25) (layer "B.Cu") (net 28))
 (segment (start 132.09905 134.0231) (end 129.27965 136.8425) (width 0.25) (layer "B.Cu") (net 28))
 (segment (start 129.27965 136.8425) (end 106.9975 136.8425) (width 0.25) (layer "B.Cu") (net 28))
 (segment (start 106.172 128.146) (end 111.503 128.146) (width 0.25) (layer "B.Cu") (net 15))
 (segment (start 111.503 128.146) (end 118.11 121.539) (width 0.25) (layer "B.Cu") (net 15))
 (segment (start 147.32 110.617) (end 147.32 110.874) (width 0.25) (layer "B.Cu") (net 20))
 (segment (start 147.32 110.874) (end 154.432 117.986) (width 0.25) (layer "B.Cu") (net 20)))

